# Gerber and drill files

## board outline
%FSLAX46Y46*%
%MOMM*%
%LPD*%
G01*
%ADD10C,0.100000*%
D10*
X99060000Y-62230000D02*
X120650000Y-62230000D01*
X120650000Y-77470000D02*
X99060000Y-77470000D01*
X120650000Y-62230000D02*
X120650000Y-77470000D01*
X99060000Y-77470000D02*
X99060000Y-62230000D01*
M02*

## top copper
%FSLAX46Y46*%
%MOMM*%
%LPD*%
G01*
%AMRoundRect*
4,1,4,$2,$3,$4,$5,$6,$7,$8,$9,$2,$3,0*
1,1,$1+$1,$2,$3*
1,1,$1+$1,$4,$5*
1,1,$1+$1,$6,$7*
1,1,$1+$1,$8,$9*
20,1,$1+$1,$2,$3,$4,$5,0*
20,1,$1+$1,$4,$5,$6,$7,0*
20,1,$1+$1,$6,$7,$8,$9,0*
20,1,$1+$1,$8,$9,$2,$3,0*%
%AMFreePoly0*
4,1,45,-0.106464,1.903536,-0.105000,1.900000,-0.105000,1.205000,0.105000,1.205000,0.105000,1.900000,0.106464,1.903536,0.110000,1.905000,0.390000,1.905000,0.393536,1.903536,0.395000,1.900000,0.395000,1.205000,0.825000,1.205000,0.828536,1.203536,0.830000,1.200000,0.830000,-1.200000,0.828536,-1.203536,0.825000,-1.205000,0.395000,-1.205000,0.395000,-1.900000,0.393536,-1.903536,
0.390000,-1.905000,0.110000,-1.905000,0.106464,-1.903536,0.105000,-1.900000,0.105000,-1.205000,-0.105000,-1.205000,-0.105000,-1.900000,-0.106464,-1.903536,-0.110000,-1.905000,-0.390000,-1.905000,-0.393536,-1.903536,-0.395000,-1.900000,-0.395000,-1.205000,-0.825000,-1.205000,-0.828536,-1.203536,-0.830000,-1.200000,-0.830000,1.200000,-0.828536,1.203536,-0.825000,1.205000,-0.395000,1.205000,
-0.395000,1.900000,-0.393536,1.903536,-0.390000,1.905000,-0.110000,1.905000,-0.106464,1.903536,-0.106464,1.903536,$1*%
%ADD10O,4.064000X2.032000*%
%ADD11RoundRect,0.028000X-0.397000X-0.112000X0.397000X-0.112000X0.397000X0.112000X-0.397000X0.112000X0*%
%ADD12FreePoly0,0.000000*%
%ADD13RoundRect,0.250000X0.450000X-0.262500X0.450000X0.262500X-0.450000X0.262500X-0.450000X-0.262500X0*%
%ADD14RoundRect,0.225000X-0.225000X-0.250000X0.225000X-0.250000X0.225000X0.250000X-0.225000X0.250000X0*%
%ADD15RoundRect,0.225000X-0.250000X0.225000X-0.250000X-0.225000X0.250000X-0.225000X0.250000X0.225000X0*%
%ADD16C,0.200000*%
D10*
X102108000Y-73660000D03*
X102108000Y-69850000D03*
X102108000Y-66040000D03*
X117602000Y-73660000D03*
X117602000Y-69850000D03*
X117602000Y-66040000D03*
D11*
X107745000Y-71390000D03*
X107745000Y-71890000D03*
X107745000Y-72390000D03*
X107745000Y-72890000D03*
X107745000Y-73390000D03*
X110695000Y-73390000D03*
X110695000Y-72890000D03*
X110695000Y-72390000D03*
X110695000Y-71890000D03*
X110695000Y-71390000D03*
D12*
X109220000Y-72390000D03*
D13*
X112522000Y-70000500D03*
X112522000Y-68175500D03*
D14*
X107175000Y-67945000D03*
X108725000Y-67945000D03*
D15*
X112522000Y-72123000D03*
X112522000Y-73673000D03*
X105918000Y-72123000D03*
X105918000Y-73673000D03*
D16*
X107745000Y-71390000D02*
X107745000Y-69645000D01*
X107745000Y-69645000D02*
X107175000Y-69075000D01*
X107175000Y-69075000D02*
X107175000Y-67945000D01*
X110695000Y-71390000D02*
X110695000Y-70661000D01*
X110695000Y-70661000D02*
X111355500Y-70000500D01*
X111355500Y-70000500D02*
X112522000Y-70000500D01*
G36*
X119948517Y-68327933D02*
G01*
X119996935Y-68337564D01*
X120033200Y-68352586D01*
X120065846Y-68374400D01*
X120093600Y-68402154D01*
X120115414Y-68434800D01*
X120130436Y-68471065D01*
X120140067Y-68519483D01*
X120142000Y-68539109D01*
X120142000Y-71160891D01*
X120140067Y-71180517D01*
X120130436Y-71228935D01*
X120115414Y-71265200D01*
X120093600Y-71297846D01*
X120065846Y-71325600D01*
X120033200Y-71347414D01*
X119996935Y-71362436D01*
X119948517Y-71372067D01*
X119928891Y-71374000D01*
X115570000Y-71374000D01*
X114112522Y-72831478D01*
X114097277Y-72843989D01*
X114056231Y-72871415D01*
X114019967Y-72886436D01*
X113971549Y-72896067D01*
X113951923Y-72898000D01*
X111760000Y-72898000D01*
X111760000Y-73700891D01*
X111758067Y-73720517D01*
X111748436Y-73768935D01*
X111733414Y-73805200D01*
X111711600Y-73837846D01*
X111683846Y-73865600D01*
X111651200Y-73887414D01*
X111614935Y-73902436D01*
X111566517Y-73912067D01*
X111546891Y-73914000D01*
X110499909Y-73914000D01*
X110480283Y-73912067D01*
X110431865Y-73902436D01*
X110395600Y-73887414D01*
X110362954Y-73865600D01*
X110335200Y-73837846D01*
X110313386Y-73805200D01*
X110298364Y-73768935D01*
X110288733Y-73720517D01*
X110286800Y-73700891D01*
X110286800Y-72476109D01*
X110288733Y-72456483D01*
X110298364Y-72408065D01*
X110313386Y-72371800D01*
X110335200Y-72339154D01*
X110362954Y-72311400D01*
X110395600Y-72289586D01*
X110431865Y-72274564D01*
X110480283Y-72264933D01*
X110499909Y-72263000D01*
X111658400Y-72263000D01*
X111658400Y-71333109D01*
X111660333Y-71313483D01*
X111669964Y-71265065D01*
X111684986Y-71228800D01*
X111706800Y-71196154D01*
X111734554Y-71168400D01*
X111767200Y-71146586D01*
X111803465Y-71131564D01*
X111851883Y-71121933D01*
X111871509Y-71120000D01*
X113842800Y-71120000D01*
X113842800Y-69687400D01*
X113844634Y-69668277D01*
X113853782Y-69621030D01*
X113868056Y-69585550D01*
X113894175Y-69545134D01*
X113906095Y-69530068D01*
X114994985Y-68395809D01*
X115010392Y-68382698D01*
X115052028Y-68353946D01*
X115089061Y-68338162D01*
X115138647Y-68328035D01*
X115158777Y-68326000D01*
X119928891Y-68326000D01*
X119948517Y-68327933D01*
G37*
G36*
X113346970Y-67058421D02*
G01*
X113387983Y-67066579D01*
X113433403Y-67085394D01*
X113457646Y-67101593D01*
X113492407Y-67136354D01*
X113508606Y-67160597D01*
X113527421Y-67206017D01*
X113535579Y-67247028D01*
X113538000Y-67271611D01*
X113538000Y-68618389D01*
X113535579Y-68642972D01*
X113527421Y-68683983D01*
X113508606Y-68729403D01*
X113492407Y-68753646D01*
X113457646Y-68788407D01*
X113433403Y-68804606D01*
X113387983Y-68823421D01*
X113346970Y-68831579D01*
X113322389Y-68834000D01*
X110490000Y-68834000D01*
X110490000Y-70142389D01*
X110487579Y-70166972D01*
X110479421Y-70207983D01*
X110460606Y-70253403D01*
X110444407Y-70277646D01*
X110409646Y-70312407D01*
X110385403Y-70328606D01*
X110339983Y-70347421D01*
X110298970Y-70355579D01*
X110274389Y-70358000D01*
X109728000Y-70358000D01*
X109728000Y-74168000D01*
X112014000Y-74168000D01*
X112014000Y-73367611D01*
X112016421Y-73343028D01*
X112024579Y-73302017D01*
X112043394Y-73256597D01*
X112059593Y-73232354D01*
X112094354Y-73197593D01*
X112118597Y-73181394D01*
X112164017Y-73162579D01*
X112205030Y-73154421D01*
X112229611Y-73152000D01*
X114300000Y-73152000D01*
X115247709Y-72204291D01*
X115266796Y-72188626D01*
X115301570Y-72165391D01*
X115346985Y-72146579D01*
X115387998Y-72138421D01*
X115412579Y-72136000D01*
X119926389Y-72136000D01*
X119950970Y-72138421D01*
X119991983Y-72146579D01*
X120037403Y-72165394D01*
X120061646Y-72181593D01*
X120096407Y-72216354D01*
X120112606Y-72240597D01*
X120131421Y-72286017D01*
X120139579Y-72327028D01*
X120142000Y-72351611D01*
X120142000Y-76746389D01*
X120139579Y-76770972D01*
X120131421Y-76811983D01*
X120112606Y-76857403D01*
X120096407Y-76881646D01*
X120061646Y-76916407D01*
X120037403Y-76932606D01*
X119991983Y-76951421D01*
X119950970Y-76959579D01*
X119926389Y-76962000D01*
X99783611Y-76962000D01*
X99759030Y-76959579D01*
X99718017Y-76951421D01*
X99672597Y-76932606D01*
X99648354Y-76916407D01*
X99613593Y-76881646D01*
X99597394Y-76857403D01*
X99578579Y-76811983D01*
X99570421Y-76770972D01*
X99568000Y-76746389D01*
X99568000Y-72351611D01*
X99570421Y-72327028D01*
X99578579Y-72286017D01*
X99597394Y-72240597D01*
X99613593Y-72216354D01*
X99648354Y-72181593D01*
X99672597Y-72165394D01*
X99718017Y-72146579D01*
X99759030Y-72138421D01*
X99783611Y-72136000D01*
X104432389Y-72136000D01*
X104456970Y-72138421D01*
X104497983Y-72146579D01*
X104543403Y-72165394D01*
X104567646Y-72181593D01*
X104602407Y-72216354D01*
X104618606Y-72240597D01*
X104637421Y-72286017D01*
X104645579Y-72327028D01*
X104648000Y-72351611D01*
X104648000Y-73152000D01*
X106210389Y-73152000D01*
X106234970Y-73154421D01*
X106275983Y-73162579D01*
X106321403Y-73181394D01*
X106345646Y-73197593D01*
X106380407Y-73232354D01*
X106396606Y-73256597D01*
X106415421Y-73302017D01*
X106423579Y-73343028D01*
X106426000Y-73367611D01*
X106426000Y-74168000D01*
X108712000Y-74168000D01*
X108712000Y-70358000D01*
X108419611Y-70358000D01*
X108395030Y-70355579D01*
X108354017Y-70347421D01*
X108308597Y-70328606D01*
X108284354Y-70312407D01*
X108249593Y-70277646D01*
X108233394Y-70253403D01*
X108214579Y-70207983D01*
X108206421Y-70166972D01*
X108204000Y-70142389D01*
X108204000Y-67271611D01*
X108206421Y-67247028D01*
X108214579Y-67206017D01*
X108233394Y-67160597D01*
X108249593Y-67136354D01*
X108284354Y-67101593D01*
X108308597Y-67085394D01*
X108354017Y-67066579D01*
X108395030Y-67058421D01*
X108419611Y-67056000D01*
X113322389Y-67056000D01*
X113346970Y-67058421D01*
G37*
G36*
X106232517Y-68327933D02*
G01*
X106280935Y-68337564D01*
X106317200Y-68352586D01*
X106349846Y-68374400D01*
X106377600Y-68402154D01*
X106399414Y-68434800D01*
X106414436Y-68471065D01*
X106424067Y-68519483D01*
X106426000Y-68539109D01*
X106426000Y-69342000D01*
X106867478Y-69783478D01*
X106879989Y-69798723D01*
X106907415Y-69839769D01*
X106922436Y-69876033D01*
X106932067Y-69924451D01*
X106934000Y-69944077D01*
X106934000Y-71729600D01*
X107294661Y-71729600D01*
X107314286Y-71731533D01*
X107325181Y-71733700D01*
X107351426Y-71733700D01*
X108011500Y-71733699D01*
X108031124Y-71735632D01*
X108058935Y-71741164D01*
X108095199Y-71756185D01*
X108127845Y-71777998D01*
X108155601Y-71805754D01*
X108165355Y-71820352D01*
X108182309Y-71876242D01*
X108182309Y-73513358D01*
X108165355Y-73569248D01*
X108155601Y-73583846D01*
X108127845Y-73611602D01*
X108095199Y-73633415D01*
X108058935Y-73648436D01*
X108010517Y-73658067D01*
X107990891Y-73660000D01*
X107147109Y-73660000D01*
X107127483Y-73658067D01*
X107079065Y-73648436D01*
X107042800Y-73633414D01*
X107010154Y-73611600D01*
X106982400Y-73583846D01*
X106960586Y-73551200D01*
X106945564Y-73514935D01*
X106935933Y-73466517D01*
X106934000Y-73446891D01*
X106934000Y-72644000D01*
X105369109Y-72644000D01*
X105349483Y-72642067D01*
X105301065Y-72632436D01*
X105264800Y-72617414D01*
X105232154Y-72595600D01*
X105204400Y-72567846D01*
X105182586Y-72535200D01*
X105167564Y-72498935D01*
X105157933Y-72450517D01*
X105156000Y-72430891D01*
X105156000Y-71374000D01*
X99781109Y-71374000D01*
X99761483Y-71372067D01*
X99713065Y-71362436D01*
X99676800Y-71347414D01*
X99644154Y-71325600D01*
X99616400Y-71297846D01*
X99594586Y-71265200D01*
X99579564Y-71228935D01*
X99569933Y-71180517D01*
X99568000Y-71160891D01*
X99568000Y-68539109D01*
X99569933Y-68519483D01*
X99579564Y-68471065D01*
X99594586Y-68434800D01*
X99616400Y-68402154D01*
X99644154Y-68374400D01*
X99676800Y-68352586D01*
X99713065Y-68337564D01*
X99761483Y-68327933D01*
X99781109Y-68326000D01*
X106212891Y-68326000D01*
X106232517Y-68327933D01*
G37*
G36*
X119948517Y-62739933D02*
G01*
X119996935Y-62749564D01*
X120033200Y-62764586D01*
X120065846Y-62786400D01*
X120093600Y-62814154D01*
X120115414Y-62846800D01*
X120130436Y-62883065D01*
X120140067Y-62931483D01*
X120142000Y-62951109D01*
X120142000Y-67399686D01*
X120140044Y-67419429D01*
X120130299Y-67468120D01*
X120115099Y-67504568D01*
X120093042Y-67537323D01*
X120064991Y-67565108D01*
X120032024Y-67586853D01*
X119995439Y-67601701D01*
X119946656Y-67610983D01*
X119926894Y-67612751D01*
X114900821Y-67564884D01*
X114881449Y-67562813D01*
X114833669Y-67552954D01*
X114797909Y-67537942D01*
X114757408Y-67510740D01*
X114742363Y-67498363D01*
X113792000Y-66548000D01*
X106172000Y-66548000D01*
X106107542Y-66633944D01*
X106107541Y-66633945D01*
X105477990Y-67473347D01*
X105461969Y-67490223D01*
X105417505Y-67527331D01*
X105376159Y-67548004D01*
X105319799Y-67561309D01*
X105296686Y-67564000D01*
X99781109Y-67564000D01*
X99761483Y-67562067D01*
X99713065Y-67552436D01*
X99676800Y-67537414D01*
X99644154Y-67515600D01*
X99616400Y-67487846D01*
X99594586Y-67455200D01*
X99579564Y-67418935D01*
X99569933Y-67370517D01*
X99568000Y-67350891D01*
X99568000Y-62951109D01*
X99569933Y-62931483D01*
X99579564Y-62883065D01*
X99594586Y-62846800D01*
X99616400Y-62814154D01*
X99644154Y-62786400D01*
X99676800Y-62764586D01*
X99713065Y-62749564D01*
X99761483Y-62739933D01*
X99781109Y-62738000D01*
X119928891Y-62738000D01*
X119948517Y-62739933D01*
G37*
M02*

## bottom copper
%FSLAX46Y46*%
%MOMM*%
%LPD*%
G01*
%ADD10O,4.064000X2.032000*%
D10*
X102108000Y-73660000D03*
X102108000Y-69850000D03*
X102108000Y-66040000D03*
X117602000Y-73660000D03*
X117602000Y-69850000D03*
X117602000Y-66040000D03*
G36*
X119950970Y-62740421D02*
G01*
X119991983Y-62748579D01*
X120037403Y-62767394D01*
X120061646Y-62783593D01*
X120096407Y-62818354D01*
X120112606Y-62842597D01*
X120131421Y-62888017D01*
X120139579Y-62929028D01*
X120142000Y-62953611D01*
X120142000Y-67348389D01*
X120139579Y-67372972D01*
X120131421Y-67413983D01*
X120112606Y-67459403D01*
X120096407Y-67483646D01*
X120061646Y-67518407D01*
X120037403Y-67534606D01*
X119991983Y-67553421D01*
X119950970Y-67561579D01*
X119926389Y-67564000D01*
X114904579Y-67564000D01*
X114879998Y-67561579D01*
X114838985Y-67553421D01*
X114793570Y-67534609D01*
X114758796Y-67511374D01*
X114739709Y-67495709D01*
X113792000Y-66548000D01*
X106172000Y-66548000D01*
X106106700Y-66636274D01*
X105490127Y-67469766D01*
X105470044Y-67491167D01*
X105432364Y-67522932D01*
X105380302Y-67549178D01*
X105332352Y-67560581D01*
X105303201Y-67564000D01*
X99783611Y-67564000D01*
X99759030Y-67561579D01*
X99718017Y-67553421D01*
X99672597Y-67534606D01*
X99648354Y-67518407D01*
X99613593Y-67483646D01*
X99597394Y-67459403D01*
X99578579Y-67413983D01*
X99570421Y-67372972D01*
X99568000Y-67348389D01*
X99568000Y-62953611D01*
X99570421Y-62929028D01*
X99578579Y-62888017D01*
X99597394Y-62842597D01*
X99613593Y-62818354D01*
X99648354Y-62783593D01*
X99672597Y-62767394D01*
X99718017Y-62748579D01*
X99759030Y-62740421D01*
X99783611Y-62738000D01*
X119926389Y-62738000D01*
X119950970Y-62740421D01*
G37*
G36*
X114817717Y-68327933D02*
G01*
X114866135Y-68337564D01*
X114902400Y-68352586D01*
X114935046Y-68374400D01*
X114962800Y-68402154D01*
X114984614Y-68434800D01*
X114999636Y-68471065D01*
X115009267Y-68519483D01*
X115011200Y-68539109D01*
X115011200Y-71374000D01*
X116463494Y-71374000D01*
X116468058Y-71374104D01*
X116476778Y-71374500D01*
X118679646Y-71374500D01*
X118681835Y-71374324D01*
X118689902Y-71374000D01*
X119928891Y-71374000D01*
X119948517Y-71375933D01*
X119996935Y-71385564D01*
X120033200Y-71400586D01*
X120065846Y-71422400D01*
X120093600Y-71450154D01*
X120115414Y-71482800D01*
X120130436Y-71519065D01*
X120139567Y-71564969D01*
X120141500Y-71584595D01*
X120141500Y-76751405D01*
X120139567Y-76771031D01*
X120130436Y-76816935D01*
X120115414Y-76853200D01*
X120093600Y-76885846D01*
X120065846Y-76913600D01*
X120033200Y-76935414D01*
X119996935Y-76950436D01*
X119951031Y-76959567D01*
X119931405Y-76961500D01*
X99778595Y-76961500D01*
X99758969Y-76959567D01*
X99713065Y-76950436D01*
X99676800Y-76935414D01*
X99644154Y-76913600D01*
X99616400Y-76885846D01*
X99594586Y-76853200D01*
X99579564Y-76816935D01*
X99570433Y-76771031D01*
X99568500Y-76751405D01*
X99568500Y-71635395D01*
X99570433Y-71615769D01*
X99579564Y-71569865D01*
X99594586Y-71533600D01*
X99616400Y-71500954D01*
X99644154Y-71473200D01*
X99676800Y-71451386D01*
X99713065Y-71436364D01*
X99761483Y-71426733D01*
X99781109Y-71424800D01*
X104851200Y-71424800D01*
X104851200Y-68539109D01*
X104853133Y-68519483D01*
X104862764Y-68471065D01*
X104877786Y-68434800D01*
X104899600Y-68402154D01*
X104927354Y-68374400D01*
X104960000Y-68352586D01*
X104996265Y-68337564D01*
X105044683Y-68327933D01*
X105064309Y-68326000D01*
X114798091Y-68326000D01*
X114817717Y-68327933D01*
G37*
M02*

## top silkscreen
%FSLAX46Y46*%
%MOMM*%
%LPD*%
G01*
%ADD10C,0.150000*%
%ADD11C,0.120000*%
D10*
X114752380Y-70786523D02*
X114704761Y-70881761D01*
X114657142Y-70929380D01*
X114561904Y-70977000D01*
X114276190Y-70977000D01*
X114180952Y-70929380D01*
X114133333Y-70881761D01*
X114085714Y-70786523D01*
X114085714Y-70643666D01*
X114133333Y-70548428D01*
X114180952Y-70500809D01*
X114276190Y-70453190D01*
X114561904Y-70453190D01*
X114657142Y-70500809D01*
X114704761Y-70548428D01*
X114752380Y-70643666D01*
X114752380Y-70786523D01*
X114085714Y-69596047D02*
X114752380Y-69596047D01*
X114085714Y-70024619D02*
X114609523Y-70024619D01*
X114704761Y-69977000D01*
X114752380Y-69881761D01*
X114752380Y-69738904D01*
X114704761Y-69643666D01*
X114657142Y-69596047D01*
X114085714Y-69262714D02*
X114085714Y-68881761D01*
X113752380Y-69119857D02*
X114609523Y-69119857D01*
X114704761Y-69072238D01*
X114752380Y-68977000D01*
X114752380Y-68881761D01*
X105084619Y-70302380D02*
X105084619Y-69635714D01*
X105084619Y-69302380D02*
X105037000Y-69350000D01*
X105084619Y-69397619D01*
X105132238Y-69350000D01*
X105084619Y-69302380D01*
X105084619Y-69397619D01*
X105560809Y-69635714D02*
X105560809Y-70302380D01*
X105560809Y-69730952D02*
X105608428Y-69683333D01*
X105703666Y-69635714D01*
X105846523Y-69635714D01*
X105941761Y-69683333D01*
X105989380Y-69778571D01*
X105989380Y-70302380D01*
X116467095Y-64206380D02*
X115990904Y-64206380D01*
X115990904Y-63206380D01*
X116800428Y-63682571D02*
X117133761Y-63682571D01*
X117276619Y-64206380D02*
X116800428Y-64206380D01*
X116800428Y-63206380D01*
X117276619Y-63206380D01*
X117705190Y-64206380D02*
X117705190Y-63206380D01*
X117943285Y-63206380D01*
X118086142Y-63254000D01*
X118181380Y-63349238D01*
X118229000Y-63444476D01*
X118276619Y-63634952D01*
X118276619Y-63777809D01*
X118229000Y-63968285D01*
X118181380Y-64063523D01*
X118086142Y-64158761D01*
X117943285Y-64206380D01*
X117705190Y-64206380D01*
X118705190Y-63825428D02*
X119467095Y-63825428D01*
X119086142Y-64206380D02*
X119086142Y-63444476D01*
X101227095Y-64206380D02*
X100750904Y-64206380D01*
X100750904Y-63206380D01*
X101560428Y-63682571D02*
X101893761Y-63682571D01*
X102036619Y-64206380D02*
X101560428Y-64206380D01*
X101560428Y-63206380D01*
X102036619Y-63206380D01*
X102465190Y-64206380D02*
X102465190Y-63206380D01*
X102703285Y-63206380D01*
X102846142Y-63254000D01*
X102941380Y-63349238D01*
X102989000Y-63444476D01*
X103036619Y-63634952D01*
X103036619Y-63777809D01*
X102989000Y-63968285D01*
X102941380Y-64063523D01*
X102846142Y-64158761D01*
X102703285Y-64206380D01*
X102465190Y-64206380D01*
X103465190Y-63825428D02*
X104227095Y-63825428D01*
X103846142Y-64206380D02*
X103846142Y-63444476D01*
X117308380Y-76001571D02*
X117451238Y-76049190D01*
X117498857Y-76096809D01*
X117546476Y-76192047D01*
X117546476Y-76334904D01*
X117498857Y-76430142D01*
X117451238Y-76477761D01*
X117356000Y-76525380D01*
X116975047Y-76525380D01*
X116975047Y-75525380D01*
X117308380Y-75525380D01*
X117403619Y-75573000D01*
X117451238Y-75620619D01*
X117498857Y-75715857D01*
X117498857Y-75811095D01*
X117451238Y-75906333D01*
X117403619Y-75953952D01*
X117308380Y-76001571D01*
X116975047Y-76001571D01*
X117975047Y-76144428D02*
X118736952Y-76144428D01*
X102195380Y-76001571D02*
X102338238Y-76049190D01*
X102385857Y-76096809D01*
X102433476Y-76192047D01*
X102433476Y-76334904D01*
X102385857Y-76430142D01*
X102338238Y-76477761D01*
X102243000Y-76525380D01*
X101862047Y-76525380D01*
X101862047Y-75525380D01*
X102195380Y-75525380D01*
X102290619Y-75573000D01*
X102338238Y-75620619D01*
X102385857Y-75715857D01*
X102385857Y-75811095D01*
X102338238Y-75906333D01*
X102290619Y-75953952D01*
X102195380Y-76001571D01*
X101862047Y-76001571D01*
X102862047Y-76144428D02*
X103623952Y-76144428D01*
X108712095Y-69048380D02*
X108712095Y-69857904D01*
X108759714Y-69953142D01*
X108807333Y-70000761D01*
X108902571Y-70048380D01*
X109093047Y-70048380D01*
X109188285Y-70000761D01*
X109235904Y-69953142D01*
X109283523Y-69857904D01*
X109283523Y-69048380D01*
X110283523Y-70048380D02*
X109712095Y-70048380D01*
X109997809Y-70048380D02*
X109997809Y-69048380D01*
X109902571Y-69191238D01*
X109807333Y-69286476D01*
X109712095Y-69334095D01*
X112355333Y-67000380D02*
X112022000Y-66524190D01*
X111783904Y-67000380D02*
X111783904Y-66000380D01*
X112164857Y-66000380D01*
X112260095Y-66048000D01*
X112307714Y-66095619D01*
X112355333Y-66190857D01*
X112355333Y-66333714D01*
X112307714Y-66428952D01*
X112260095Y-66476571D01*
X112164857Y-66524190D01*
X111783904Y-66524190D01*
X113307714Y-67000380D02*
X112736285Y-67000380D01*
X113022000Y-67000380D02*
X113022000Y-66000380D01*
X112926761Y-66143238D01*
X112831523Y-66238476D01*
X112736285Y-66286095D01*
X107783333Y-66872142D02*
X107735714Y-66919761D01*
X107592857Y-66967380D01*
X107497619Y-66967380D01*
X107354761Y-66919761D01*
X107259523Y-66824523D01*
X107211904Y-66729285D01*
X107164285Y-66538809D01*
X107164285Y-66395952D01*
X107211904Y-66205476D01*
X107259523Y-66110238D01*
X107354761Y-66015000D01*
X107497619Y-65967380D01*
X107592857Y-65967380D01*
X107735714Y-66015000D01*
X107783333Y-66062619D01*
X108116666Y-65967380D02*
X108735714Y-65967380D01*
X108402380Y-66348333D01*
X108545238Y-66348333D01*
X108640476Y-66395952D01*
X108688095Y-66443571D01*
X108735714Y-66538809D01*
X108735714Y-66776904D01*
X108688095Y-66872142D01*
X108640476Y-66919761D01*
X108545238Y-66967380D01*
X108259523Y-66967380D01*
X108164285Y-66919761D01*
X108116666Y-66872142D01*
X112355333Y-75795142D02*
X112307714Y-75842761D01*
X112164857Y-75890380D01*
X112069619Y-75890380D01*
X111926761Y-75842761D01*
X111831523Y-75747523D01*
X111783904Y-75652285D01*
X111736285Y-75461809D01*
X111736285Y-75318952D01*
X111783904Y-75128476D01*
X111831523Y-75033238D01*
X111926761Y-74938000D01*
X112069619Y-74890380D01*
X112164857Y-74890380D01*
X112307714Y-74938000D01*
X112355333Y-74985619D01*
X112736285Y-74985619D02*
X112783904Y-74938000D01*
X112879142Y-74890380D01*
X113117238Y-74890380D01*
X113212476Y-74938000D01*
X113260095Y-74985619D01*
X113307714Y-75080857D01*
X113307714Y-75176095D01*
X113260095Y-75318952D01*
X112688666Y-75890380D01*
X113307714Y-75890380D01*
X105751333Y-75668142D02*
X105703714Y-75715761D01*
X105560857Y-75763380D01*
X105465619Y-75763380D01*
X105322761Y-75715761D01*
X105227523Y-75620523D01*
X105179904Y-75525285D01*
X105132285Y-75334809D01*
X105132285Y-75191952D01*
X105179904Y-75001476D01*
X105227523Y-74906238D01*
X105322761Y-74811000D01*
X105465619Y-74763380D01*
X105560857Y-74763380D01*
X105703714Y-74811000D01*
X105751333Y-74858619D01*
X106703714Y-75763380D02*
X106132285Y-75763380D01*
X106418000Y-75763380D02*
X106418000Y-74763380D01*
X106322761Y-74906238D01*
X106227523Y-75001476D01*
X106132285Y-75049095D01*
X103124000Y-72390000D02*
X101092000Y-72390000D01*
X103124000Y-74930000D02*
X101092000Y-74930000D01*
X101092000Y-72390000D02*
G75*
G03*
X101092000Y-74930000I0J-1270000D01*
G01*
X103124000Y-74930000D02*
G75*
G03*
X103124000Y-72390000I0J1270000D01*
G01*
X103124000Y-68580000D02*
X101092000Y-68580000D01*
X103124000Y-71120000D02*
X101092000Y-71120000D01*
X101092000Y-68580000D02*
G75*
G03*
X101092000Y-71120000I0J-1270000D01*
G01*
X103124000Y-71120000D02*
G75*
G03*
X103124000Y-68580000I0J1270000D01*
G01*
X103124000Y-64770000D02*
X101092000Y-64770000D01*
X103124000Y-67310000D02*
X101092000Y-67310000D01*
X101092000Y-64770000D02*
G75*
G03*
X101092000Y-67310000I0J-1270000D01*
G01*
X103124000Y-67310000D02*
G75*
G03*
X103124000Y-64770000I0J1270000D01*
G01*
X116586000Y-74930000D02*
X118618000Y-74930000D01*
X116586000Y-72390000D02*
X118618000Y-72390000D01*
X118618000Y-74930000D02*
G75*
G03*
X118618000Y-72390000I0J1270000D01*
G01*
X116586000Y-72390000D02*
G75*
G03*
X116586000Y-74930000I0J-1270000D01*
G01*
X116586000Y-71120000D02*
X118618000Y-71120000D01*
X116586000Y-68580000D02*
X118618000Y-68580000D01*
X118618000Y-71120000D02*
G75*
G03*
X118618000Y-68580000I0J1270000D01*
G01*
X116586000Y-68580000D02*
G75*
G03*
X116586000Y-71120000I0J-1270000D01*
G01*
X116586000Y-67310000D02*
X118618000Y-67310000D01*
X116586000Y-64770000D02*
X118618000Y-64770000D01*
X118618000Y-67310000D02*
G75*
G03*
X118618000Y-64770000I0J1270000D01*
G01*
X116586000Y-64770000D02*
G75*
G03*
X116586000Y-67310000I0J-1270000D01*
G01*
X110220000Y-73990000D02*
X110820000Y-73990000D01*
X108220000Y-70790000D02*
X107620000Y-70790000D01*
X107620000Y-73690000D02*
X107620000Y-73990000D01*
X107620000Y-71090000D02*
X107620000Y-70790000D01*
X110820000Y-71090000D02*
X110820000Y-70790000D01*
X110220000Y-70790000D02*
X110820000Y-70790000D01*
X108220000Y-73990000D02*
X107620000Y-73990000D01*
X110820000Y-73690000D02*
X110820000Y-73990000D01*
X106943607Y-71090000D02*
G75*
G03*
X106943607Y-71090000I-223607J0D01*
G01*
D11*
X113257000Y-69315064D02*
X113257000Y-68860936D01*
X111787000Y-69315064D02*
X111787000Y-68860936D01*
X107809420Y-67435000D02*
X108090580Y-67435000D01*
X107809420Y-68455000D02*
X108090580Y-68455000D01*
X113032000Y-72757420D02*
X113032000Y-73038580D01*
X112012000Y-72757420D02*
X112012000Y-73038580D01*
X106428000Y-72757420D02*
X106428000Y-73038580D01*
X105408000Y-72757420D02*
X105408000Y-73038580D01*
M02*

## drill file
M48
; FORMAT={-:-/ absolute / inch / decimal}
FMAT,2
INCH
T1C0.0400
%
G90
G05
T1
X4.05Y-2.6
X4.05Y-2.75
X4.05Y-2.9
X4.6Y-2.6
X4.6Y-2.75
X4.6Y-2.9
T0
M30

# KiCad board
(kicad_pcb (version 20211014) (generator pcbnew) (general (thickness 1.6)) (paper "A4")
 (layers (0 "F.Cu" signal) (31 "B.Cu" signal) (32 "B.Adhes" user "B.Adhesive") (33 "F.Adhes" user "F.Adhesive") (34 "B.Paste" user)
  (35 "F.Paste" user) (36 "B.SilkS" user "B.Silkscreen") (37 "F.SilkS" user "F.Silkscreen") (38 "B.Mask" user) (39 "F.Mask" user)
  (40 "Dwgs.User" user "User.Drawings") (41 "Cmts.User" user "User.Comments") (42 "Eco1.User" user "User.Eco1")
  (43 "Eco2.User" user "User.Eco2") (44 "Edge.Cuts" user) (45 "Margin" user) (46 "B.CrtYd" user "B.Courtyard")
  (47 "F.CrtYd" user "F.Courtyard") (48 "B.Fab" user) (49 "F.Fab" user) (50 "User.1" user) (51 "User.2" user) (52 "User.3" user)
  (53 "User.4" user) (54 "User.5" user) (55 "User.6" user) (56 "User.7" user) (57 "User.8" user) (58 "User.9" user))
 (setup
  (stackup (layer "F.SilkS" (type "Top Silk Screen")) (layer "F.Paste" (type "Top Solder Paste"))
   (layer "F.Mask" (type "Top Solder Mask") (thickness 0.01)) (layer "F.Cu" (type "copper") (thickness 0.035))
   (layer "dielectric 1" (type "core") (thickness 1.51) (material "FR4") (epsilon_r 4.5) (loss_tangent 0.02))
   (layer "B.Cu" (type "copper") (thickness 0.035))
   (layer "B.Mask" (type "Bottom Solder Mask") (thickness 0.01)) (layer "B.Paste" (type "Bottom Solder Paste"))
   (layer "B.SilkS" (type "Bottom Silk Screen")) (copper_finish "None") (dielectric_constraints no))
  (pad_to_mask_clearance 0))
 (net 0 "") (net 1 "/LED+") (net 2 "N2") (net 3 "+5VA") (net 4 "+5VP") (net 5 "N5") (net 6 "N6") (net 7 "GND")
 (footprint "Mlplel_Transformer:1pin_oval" (layer "F.Cu") (at 116.84 66.04)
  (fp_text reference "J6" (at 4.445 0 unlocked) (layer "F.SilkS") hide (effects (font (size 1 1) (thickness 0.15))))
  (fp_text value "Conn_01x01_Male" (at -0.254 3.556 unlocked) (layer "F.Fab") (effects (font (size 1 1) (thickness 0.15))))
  (fp_line (start -0.254 1.27) (end 1.778 1.27) (layer "F.SilkS") (width 0.15))
  (fp_line (start -0.254 -1.27) (end 1.778 -1.27) (layer "F.SilkS") (width 0.15))
  (fp_arc (start 1.778 -1.27) (mid 3.048 0) (end 1.778 1.27) (layer "F.SilkS") (width 0.15))
  (fp_arc (start -0.254 1.27) (mid -1.524 0) (end -0.254 -1.27) (layer "F.SilkS") (width 0.15))
  (pad "1" thru_hole oval (at 0 0) (size 4.064 2.032) (drill 1.016 (offset 0.762 0)) (layers *.Cu *.Mask) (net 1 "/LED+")))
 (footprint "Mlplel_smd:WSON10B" (layer "F.Cu") (at 109.22 72.39)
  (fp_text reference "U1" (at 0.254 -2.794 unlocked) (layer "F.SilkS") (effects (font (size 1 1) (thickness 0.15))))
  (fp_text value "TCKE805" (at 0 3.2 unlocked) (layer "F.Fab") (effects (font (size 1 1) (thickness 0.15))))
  (fp_line (start 1 1.6) (end 1.6 1.6) (layer "F.SilkS") (width 0.15))
  (fp_line (start -1 -1.6) (end -1.6 -1.6) (layer "F.SilkS") (width 0.15))
  (fp_line (start -1.6 1.3) (end -1.6 1.6) (layer "F.SilkS") (width 0.15))
  (fp_line (start -1.6 -1.3) (end -1.6 -1.6) (layer "F.SilkS") (width 0.15))
  (fp_line (start 1.6 -1.3) (end 1.6 -1.6) (layer "F.SilkS") (width 0.15))
  (fp_line (start 1 -1.6) (end 1.6 -1.6) (layer "F.SilkS") (width 0.15))
  (fp_line (start -1 1.6) (end -1.6 1.6) (layer "F.SilkS") (width 0.15))
  (fp_line (start 1.6 1.3) (end 1.6 1.6) (layer "F.SilkS") (width 0.15))
  (fp_circle (center -2.5 -1.3) (end -2.3 -1.2) (layer "F.SilkS") (width 0.15) (fill none))
  (pad "1" smd roundrect (at -1.475 -1) (size 0.85 0.28) (layers "F.Cu" "F.Paste" "F.Mask") (roundrect_rratio 0.1) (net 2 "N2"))
  (pad "2" smd roundrect (at -1.475 -0.5) (size 0.85 0.28) (layers "F.Cu" "F.Paste" "F.Mask") (roundrect_rratio 0.1) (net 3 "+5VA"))
  (pad "3" smd roundrect (at -1.475 0) (size 0.85 0.28) (layers "F.Cu" "F.Paste" "F.Mask") (roundrect_rratio 0.1) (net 3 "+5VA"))
  (pad "4" smd roundrect (at -1.475 0.5) (size 0.85 0.28) (layers "F.Cu" "F.Paste" "F.Mask") (roundrect_rratio 0.1) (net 3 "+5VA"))
  (pad "5" smd roundrect (at -1.475 1) (size 0.85 0.28) (layers "F.Cu" "F.Paste" "F.Mask") (roundrect_rratio 0.1) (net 3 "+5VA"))
  (pad "6" smd roundrect (at 1.475 1) (size 0.85 0.28) (layers "F.Cu" "F.Paste" "F.Mask") (roundrect_rratio 0.1) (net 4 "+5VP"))
  (pad "7" smd roundrect (at 1.475 0.5) (size 0.85 0.28) (layers "F.Cu" "F.Paste" "F.Mask") (roundrect_rratio 0.1) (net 4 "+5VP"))
  (pad "8" smd roundrect (at 1.475 0) (size 0.85 0.28) (layers "F.Cu" "F.Paste" "F.Mask") (roundrect_rratio 0.1) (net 4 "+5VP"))
  (pad "9" smd roundrect (at 1.475 -0.5) (size 0.85 0.28) (layers "F.Cu" "F.Paste" "F.Mask") (roundrect_rratio 0.1) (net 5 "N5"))
  (pad "10" smd roundrect (at 1.475 -1) (size 0.85 0.28) (layers "F.Cu" "F.Paste" "F.Mask") (roundrect_rratio 0.1) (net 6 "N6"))
  (pad "11" smd custom (at 0 0) (size 0.85 0.28) (layers "F.Cu" "F.Paste" "F.Mask") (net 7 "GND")
   (options (clearance outline) (anchor rect)) (primitives)))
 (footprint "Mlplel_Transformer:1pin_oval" (layer "F.Cu") (at 116.84 73.66)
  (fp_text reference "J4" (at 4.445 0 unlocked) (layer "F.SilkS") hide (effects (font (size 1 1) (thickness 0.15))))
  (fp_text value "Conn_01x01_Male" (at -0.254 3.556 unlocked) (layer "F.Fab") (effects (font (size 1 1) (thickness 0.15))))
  (fp_line (start -0.254 -1.27) (end 1.778 -1.27) (layer "F.SilkS") (width 0.15))
  (fp_line (start -0.254 1.27) (end 1.778 1.27) (layer "F.SilkS") (width 0.15))
  (fp_arc (start 1.778 -1.27) (mid 3.048 0) (end 1.778 1.27) (layer "F.SilkS") (width 0.15))
  (fp_arc (start -0.254 1.27) (mid -1.524 0) (end -0.254 -1.27) (layer "F.SilkS") (width 0.15))
  (pad "1" thru_hole oval (at 0 0) (size 4.064 2.032) (drill 1.016 (offset 0.762 0)) (layers *.Cu *.Mask) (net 7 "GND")))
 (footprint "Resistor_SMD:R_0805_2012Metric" (layer "F.Cu") (at 112.522 69.088 90)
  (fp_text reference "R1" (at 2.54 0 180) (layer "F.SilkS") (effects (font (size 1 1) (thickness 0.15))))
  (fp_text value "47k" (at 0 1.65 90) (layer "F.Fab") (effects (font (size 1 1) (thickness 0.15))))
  (fp_line (start -0.227064 0.735) (end 0.227064 0.735) (layer "F.SilkS") (width 0.12))
  (fp_line (start -0.227064 -0.735) (end 0.227064 -0.735) (layer "F.SilkS") (width 0.12))
  (pad "1" smd roundrect (at -0.9125 0 90) (size 1.025 1.4) (layers "F.Cu" "F.Paste" "F.Mask") (roundrect_rratio 0.243902439) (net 6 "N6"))
  (pad "2" smd roundrect (at 0.9125 0 90) (size 1.025 1.4) (layers "F.Cu" "F.Paste" "F.Mask") (roundrect_rratio 0.243902439) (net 7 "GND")))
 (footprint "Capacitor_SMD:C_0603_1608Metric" (layer "F.Cu") (at 107.95 67.945)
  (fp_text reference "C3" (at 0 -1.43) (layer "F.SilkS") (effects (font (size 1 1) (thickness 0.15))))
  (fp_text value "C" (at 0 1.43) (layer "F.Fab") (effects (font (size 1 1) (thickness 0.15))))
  (fp_line (start -0.14058 -0.51) (end 0.14058 -0.51) (layer "F.SilkS") (width 0.12))
  (fp_line (start -0.14058 0.51) (end 0.14058 0.51) (layer "F.SilkS") (width 0.12))
  (pad "1" smd roundrect (at -0.775 0) (size 0.9 0.95) (layers "F.Cu" "F.Paste" "F.Mask") (roundrect_rratio 0.25) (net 2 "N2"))
  (pad "2" smd roundrect (at 0.775 0) (size 0.9 0.95) (layers "F.Cu" "F.Paste" "F.Mask") (roundrect_rratio 0.25) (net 7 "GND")))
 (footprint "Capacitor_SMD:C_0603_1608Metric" (layer "F.Cu") (at 112.522 72.898 -90)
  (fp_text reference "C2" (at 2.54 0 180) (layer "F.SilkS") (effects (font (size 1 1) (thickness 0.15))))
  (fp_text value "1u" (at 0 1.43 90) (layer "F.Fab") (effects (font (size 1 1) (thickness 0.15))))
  (fp_line (start -0.14058 -0.51) (end 0.14058 -0.51) (layer "F.SilkS") (width 0.12))
  (fp_line (start -0.14058 0.51) (end 0.14058 0.51) (layer "F.SilkS") (width 0.12))
  (pad "1" smd roundrect (at -0.775 0 270) (size 0.9 0.95) (layers "F.Cu" "F.Paste" "F.Mask") (roundrect_rratio 0.25) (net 4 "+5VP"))
  (pad "2" smd roundrect (at 0.775 0 270) (size 0.9 0.95) (layers "F.Cu" "F.Paste" "F.Mask") (roundrect_rratio 0.25) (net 7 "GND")))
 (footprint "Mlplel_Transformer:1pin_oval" (layer "F.Cu") (at 102.87 73.66 180)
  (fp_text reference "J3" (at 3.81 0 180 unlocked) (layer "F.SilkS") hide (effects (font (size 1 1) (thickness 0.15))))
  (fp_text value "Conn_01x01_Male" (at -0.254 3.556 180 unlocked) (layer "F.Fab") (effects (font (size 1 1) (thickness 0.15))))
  (fp_line (start -0.254 -1.27) (end 1.778 -1.27) (layer "F.SilkS") (width 0.15))
  (fp_line (start -0.254 1.27) (end 1.778 1.27) (layer "F.SilkS") (width 0.15))
  (fp_arc (start -0.254 1.27) (mid -1.524 0) (end -0.254 -1.27) (layer "F.SilkS") (width 0.15))
  (fp_arc (start 1.778 -1.27) (mid 3.048 0) (end 1.778 1.27) (layer "F.SilkS") (width 0.15))
  (pad "1" thru_hole oval (at 0 0 180) (size 4.064 2.032) (drill 1.016 (offset 0.762 0)) (layers *.Cu *.Mask) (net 7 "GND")))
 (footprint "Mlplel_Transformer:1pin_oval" (layer "F.Cu") (at 102.87 69.85 180)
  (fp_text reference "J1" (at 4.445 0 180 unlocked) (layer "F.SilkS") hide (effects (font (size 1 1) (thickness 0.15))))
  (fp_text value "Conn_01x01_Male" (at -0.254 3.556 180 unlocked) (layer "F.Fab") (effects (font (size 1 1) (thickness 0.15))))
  (fp_line (start -0.254 1.27) (end 1.778 1.27) (layer "F.SilkS") (width 0.15))
  (fp_line (start -0.254 -1.27) (end 1.778 -1.27) (layer "F.SilkS") (width 0.15))
  (fp_arc (start 1.778 -1.27) (mid 3.048 0) (end 1.778 1.27) (layer "F.SilkS") (width 0.15))
  (fp_arc (start -0.254 1.27) (mid -1.524 0) (end -0.254 -1.27) (layer "F.SilkS") (width 0.15))
  (pad "1" thru_hole oval (at 0 0 180) (size 4.064 2.032) (drill 1.016 (offset 0.762 0)) (layers *.Cu *.Mask) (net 3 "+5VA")))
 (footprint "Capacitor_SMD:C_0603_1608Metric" (layer "F.Cu") (at 105.918 72.898 -90)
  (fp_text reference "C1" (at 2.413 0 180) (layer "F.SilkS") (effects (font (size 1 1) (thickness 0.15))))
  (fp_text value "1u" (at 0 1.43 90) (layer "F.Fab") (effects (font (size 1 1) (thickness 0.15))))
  (fp_line (start -0.14058 -0.51) (end 0.14058 -0.51) (layer "F.SilkS") (width 0.12))
  (fp_line (start -0.14058 0.51) (end 0.14058 0.51) (layer "F.SilkS") (width 0.12))
  (pad "1" smd roundrect (at -0.775 0 270) (size 0.9 0.95) (layers "F.Cu" "F.Paste" "F.Mask") (roundrect_rratio 0.25) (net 3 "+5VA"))
  (pad "2" smd roundrect (at 0.775 0 270) (size 0.9 0.95) (layers "F.Cu" "F.Paste" "F.Mask") (roundrect_rratio 0.25) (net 7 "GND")))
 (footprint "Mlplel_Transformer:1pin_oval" (layer "F.Cu") (at 116.84 69.85)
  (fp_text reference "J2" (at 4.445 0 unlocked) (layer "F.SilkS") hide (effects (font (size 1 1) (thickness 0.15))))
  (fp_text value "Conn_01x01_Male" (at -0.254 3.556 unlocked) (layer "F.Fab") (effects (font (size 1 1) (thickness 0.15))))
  (fp_line (start -0.254 1.27) (end 1.778 1.27) (layer "F.SilkS") (width 0.15))
  (fp_line (start -0.254 -1.27) (end 1.778 -1.27) (layer "F.SilkS") (width 0.15))
  (fp_arc (start -0.254 1.27) (mid -1.524 0) (end -0.254 -1.27) (layer "F.SilkS") (width 0.15))
  (fp_arc (start 1.778 -1.27) (mid 3.048 0) (end 1.778 1.27) (layer "F.SilkS") (width 0.15))
  (pad "1" thru_hole oval (at 0 0) (size 4.064 2.032) (drill 1.016 (offset 0.762 0)) (layers *.Cu *.Mask) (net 4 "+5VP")))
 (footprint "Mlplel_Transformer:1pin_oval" (layer "F.Cu") (at 102.87 66.04 180)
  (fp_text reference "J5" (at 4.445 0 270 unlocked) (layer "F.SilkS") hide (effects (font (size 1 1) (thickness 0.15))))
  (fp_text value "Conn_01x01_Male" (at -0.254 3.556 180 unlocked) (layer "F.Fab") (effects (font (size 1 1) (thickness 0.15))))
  (fp_line (start -0.254 -1.27) (end 1.778 -1.27) (layer "F.SilkS") (width 0.15))
  (fp_line (start -0.254 1.27) (end 1.778 1.27) (layer "F.SilkS") (width 0.15))
  (fp_arc (start -0.254 1.27) (mid -1.524 0) (end -0.254 -1.27) (layer "F.SilkS") (width 0.15))
  (fp_arc (start 1.778 -1.27) (mid 3.048 0) (end 1.778 1.27) (layer "F.SilkS") (width 0.15))
  (pad "1" thru_hole oval (at 0 0 180) (size 4.064 2.032) (drill 1.016 (offset 0.762 0)) (layers *.Cu *.Mask) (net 1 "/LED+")))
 (gr_line (start 99.06 62.23) (end 120.65 62.23) (layer "Edge.Cuts") (width 0.1))
 (gr_line (start 120.65 77.47) (end 99.06 77.47) (layer "Edge.Cuts") (width 0.1))
 (gr_line (start 120.65 62.23) (end 120.65 77.47) (layer "Edge.Cuts") (width 0.1))
 (gr_line (start 99.06 77.47) (end 99.06 62.23) (layer "Edge.Cuts") (width 0.1))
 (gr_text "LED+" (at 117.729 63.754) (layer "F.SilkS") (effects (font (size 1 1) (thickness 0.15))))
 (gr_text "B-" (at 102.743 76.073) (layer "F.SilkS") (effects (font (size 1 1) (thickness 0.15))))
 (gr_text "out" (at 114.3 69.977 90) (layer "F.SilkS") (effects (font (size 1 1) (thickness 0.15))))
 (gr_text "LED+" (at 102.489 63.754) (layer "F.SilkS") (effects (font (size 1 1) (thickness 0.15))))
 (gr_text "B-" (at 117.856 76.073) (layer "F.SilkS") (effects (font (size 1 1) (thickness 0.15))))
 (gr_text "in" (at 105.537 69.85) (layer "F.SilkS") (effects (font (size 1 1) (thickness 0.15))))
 (segment (start 107.175 69.075) (end 107.175 67.945) (width 0.2) (layer "F.Cu") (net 2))
 (segment (start 107.745 71.39) (end 107.745 69.645) (width 0.2) (layer "F.Cu") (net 2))
 (segment (start 107.745 69.645) (end 107.175 69.075) (width 0.2) (layer "F.Cu") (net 2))
 (segment (start 111.3555 70.0005) (end 112.522 70.0005) (width 0.2) (layer "F.Cu") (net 6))
 (segment (start 110.695 71.39) (end 110.695 70.661) (width 0.2) (layer "F.Cu") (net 6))
 (segment (start 110.695 70.661) (end 111.3555 70.0005) (width 0.2) (layer "F.Cu") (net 6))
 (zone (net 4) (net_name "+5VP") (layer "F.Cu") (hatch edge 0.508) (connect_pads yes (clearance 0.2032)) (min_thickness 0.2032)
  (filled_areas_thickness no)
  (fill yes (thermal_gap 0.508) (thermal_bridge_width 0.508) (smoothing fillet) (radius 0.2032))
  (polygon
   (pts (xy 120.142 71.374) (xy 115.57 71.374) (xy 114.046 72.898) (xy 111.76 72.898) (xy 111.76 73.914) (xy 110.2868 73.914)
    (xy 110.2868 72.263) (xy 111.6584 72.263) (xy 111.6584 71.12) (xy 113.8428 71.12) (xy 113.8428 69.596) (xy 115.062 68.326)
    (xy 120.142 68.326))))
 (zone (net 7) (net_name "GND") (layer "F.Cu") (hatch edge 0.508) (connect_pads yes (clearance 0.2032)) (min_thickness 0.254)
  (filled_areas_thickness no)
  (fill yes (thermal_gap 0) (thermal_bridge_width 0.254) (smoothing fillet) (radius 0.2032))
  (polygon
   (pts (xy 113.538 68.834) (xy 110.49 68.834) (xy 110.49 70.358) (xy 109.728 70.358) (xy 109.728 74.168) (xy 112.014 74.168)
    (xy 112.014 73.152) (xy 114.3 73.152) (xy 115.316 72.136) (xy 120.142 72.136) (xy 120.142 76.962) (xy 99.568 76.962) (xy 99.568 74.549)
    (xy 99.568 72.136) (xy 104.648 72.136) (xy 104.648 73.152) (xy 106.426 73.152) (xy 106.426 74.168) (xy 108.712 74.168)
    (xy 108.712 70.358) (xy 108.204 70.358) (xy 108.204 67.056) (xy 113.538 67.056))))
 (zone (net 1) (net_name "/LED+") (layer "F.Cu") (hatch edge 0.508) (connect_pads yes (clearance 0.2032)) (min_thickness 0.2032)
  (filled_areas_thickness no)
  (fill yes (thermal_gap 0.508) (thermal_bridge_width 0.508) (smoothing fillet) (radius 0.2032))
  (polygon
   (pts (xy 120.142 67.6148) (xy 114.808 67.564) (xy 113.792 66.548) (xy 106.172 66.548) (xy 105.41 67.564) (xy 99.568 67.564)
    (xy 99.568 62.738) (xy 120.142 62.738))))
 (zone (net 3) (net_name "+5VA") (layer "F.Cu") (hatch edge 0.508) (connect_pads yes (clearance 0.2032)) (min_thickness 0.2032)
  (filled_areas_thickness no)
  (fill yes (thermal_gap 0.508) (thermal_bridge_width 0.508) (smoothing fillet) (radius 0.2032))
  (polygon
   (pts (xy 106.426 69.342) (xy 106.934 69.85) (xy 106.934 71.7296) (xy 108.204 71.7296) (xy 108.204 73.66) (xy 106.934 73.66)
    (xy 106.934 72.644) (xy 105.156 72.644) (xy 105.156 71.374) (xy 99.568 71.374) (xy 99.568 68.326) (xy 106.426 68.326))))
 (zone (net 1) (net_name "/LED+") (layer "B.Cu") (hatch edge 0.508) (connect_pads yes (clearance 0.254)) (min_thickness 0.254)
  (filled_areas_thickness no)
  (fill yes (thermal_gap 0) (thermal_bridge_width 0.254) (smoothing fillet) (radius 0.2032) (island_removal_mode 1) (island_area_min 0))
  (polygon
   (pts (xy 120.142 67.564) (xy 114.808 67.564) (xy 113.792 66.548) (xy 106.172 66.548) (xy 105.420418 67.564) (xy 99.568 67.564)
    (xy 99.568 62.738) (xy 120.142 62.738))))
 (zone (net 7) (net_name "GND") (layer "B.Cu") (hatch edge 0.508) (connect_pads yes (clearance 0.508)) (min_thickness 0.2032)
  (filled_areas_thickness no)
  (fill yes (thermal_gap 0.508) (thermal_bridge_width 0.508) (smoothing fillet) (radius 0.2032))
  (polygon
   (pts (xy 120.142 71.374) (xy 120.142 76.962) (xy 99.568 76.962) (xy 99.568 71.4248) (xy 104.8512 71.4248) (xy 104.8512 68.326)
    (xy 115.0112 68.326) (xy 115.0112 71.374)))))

